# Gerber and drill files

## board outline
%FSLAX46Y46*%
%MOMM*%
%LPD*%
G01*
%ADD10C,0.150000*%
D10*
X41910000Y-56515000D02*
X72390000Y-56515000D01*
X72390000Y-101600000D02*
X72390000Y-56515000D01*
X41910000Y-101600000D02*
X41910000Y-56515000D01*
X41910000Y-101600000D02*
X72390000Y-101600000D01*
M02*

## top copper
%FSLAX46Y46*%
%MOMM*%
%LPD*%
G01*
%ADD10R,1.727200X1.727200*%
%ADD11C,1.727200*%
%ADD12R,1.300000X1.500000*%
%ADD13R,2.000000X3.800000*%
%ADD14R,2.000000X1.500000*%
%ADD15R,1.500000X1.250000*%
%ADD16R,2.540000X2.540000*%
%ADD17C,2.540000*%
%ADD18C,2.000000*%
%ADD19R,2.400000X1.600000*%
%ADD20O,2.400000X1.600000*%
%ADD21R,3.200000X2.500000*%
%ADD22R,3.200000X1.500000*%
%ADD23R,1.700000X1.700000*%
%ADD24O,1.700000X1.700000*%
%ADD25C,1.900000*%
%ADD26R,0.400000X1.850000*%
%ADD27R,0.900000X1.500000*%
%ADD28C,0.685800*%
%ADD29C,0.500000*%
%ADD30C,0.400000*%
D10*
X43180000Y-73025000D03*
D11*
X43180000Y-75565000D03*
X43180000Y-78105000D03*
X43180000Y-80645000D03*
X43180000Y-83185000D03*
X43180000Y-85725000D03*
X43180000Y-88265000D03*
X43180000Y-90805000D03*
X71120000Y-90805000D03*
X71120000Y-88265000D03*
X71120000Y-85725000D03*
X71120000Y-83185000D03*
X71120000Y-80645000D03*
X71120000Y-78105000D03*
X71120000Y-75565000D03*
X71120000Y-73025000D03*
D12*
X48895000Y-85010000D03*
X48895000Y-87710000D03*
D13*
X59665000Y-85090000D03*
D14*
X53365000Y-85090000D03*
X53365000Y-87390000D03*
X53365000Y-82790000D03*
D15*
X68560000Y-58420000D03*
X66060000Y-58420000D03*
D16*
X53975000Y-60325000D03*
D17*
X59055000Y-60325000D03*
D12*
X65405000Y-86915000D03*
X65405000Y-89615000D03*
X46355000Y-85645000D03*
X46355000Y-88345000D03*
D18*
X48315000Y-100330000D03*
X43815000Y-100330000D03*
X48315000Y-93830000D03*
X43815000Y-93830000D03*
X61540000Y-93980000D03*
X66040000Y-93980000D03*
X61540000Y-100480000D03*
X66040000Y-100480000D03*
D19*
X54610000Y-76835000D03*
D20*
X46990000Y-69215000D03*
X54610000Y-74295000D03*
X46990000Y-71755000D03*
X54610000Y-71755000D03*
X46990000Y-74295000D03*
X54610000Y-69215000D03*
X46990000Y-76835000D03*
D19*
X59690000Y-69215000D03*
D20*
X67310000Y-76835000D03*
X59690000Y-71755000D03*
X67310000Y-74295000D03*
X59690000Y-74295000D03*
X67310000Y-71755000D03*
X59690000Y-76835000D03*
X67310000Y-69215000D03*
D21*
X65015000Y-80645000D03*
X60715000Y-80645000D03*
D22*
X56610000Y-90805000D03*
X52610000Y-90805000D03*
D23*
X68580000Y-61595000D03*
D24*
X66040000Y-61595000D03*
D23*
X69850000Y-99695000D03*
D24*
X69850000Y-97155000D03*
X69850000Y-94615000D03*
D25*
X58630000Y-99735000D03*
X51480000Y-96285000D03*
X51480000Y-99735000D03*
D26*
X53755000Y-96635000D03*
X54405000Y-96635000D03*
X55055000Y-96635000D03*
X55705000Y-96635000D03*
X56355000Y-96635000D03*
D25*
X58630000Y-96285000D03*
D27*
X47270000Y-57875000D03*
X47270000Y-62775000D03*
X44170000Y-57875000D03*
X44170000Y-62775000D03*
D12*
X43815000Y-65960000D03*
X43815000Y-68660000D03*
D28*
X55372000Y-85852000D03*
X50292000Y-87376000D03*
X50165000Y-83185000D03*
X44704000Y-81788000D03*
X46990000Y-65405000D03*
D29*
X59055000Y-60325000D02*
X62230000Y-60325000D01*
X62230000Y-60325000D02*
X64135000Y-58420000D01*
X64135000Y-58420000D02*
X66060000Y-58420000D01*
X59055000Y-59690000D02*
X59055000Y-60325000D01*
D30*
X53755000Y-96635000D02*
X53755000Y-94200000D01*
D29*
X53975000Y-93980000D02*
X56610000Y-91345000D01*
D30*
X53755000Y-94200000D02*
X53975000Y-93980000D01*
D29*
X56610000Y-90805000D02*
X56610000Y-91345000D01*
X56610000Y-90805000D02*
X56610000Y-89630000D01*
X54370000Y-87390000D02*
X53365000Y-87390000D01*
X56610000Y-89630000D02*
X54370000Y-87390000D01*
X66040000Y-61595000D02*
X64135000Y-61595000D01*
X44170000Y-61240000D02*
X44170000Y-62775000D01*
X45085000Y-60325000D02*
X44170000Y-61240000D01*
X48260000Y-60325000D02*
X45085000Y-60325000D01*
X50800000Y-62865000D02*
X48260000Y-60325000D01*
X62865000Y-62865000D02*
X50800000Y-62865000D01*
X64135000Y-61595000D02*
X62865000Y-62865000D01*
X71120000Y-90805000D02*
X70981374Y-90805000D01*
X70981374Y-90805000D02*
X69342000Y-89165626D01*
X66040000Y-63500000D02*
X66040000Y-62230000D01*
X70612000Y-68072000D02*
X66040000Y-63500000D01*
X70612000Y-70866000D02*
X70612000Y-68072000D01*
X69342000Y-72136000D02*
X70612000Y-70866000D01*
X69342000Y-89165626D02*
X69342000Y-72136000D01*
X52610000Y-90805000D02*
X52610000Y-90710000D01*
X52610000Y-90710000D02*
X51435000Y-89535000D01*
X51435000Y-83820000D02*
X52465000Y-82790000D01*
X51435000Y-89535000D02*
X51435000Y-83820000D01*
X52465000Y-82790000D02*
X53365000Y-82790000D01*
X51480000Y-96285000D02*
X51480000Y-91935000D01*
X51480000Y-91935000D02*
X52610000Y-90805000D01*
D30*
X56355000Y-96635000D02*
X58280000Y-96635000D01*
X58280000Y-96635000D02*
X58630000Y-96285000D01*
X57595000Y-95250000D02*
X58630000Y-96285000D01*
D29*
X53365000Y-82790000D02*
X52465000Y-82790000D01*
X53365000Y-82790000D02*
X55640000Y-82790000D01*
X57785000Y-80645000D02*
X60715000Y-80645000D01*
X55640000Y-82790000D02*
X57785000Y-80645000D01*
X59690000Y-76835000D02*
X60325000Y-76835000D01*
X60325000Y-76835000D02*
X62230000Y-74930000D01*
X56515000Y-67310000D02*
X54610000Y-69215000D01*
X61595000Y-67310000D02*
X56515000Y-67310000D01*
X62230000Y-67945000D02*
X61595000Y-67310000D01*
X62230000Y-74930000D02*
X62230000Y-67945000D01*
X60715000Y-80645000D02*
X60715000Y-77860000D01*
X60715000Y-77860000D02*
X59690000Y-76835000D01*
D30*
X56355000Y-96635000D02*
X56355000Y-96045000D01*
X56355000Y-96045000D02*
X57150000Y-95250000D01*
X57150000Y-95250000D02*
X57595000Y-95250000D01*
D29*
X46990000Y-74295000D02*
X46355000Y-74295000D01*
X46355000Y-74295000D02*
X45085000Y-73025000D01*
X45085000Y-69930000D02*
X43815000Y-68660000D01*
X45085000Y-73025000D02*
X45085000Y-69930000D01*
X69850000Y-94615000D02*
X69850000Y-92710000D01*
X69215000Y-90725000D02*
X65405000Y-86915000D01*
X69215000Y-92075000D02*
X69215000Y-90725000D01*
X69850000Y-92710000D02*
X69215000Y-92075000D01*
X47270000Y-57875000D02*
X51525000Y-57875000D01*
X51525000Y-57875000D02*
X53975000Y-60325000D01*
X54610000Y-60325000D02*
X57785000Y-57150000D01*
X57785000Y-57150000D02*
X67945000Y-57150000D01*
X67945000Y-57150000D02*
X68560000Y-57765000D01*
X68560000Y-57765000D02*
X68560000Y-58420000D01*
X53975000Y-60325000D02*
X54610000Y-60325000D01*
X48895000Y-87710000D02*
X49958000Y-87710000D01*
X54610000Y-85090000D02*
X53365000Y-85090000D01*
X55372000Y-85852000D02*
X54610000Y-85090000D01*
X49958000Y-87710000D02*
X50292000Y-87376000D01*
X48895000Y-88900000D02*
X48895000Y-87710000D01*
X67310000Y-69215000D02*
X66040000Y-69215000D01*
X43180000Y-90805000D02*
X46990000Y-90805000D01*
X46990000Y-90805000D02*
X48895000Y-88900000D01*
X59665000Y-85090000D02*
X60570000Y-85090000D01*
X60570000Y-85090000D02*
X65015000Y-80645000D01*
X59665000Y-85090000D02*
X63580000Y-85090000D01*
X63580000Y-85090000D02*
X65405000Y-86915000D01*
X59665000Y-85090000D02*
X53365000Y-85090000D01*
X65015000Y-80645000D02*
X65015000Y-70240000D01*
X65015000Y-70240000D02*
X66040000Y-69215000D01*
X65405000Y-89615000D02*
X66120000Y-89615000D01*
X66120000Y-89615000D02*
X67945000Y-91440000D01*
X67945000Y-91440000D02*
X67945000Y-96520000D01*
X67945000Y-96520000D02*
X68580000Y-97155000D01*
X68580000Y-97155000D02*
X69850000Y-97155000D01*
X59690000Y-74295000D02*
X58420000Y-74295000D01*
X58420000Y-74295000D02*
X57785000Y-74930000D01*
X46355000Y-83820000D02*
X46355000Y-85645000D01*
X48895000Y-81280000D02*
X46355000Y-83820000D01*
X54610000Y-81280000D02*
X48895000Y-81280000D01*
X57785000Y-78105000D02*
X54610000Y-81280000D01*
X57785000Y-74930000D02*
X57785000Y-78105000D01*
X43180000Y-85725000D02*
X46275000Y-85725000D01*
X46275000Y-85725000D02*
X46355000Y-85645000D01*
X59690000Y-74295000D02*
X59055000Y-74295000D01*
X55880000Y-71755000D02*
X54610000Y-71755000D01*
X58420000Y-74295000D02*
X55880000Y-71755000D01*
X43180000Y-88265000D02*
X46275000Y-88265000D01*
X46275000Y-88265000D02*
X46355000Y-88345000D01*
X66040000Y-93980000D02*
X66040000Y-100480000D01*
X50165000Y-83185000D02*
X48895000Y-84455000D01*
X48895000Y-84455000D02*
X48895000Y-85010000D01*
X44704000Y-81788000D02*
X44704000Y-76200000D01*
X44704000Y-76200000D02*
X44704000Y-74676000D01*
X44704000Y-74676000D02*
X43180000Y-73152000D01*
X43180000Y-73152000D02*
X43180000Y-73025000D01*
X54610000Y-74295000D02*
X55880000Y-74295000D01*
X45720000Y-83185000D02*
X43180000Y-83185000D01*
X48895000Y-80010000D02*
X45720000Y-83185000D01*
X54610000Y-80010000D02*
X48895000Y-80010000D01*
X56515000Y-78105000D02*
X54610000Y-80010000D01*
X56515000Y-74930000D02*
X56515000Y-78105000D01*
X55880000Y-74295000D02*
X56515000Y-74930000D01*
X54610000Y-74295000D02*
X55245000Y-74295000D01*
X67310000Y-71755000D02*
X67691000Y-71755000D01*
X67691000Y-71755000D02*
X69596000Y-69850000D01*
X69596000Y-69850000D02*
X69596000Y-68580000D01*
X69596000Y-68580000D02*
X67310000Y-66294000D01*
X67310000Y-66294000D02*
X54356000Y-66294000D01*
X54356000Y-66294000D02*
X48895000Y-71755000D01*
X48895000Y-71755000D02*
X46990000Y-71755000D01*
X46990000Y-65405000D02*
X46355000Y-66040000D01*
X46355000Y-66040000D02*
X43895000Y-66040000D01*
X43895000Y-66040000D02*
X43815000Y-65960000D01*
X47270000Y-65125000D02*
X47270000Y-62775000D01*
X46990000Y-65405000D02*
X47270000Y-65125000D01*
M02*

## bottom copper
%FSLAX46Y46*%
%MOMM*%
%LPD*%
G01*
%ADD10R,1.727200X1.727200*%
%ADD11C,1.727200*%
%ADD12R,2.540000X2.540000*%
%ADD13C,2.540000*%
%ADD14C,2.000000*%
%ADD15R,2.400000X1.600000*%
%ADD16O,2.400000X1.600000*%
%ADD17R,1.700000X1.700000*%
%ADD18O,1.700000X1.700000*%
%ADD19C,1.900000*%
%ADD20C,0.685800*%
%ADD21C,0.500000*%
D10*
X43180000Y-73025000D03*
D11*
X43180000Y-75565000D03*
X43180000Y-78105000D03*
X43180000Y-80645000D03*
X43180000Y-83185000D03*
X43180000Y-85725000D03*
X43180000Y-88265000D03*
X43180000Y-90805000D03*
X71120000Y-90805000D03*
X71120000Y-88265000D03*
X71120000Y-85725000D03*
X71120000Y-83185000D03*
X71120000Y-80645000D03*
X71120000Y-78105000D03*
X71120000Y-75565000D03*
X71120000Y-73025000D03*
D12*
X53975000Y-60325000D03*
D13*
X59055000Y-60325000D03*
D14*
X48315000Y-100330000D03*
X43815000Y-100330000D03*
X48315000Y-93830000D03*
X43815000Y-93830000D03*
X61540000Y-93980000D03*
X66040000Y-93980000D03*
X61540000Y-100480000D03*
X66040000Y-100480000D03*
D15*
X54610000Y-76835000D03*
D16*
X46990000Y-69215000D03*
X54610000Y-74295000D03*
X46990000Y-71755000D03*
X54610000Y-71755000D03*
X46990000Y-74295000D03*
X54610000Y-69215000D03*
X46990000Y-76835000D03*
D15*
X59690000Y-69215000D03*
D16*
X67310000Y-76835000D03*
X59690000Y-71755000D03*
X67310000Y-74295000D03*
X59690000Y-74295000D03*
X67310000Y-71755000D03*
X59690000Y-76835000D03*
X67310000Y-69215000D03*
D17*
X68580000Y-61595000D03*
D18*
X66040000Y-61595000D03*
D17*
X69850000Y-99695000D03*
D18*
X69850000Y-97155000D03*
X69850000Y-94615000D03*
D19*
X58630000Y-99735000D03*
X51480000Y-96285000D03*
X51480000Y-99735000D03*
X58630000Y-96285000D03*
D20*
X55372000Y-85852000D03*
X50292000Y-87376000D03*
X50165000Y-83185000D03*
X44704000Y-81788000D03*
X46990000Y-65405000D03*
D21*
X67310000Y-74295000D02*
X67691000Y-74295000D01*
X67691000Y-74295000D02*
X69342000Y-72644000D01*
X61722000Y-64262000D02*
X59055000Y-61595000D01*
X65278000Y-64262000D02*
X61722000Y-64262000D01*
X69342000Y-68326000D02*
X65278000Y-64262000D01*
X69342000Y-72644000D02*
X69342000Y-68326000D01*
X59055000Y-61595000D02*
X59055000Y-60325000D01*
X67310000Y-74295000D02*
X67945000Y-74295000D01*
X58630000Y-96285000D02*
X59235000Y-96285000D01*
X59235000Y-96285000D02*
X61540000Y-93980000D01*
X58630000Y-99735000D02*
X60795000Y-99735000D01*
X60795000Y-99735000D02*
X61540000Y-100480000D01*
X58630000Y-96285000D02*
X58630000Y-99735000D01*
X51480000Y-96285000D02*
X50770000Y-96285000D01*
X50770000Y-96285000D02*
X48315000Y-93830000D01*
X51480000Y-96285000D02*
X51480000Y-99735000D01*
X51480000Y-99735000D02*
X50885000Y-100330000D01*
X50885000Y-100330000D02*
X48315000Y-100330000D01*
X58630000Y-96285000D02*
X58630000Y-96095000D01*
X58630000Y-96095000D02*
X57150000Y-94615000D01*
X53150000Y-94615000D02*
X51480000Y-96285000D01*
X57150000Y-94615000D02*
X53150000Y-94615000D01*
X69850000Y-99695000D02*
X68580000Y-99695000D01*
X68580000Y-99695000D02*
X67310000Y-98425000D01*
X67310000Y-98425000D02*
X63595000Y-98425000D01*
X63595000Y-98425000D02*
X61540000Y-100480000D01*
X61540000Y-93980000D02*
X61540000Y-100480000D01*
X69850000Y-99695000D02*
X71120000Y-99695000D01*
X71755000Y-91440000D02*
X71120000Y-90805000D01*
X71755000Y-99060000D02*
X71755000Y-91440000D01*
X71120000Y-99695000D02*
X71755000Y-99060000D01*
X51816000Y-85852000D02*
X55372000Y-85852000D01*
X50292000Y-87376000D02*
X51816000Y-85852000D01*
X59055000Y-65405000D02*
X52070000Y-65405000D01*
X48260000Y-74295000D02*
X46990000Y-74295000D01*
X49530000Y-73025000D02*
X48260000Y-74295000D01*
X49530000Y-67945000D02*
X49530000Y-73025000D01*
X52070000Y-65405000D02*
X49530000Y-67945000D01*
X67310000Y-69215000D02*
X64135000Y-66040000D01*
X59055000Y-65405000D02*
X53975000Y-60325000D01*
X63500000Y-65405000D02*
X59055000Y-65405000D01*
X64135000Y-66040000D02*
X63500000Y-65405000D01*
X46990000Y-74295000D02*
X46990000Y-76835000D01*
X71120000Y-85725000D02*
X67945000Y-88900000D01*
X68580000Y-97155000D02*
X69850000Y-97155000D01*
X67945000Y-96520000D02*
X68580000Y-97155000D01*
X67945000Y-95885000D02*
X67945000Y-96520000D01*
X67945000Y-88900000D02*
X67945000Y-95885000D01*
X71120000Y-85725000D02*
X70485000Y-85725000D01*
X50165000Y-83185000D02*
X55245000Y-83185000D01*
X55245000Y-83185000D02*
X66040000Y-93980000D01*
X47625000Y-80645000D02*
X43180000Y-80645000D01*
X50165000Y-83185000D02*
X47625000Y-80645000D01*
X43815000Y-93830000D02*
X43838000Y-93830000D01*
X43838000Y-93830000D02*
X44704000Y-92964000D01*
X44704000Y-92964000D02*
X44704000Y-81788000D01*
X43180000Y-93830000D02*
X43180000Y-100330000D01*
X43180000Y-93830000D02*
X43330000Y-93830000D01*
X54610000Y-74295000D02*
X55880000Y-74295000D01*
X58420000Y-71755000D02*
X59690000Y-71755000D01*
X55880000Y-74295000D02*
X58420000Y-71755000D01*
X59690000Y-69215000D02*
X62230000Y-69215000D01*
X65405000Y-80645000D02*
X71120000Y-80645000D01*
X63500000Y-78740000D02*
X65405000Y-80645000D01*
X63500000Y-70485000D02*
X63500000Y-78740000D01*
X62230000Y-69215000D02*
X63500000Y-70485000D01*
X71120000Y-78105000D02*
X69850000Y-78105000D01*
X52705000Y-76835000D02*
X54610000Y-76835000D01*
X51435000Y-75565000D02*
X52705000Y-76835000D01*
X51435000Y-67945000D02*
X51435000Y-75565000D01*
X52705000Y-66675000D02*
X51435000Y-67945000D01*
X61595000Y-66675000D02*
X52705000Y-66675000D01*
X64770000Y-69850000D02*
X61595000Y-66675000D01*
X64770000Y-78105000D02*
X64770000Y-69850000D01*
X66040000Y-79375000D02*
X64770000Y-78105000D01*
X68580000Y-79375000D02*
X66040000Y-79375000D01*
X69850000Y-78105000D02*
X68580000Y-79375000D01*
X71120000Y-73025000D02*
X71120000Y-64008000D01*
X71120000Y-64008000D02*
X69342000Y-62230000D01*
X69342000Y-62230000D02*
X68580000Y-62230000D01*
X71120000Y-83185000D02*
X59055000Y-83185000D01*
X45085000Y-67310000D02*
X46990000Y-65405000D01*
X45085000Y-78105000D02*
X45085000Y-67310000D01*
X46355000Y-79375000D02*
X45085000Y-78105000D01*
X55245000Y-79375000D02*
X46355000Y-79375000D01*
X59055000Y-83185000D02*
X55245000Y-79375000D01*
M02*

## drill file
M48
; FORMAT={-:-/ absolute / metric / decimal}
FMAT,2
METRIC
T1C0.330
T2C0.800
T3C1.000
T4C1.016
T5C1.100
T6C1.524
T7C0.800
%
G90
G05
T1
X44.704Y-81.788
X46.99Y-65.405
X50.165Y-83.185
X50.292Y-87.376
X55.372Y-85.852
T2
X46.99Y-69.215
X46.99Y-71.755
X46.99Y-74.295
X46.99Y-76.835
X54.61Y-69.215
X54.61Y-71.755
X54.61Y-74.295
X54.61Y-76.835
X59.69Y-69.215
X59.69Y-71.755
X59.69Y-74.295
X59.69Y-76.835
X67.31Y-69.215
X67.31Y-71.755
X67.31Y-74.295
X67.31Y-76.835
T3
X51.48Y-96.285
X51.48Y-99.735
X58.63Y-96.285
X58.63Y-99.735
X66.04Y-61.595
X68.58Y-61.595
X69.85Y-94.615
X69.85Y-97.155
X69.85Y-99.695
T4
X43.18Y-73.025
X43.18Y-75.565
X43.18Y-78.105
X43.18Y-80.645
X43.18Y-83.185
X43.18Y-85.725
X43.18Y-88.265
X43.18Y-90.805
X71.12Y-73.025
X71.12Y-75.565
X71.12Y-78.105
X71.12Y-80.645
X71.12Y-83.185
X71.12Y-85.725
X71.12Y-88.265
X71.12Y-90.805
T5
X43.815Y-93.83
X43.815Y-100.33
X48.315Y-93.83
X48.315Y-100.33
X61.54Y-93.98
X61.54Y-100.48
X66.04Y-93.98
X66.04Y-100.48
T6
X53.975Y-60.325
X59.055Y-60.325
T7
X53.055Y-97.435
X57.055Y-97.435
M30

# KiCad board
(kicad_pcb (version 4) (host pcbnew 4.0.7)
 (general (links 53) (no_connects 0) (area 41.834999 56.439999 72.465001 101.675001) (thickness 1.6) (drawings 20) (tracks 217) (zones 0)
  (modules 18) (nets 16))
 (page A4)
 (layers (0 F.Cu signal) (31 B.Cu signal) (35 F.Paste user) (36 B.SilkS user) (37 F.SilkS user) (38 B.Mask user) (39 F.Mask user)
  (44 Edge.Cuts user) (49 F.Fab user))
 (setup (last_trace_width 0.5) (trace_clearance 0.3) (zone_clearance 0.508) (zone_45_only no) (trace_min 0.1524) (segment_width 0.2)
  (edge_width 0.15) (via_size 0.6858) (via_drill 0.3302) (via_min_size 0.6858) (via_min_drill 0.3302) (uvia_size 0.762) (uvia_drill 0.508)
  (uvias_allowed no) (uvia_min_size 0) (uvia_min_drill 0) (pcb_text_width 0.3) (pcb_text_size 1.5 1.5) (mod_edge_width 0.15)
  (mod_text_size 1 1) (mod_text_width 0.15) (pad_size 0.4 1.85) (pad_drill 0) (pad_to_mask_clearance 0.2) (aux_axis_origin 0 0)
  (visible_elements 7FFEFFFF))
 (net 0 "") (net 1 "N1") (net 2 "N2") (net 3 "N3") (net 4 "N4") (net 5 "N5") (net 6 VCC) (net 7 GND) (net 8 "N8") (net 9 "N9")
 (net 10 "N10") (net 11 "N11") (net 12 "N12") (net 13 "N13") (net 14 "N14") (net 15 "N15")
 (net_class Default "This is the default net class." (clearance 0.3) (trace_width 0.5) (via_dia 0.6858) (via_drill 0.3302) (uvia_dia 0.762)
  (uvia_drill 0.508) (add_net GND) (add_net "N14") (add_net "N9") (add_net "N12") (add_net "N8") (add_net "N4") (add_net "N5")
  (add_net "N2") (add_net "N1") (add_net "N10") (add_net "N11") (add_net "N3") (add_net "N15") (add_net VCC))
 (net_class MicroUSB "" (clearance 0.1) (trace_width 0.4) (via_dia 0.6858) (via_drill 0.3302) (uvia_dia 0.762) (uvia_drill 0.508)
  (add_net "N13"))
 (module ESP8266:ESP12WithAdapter (layer F.Cu) (at 41.91 92.075)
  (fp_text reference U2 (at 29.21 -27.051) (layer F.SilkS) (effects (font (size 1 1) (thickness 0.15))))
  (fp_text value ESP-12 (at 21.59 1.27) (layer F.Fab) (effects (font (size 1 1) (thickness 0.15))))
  (pad 1 thru_hole rect (at 1.27 -19.05) (size 1.7272 1.7272) (drill 1.016) (layers *.Cu *.Mask F.SilkS) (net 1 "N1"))
  (pad 2 thru_hole circle (at 1.27 -16.51) (size 1.7272 1.7272) (drill 1.016) (layers *.Cu *.Mask F.SilkS))
  (pad 3 thru_hole circle (at 1.27 -13.97) (size 1.7272 1.7272) (drill 1.016) (layers *.Cu *.Mask F.SilkS))
  (pad 4 thru_hole circle (at 1.27 -11.43) (size 1.7272 1.7272) (drill 1.016) (layers *.Cu *.Mask F.SilkS) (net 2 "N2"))
  (pad 5 thru_hole circle (at 1.27 -8.89) (size 1.7272 1.7272) (drill 1.016) (layers *.Cu *.Mask F.SilkS) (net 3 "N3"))
  (pad 6 thru_hole circle (at 1.27 -6.35) (size 1.7272 1.7272) (drill 1.016) (layers *.Cu *.Mask F.SilkS) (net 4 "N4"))
  (pad 7 thru_hole circle (at 1.27 -3.81) (size 1.7272 1.7272) (drill 1.016) (layers *.Cu *.Mask F.SilkS) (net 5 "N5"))
  (pad 8 thru_hole circle (at 1.27 -1.27) (size 1.7272 1.7272) (drill 1.016) (layers *.Cu *.Mask F.SilkS) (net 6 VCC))
  (pad 9 thru_hole circle (at 29.21 -1.27) (size 1.7272 1.7272) (drill 1.016) (layers *.Cu *.Mask F.SilkS) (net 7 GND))
  (pad 10 thru_hole circle (at 29.21 -3.81) (size 1.7272 1.7272) (drill 1.016) (layers *.Cu *.Mask F.SilkS))
  (pad 11 thru_hole circle (at 29.21 -6.35) (size 1.7272 1.7272) (drill 1.016) (layers *.Cu *.Mask F.SilkS) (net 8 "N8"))
  (pad 12 thru_hole circle (at 29.21 -8.89) (size 1.7272 1.7272) (drill 1.016) (layers *.Cu *.Mask F.SilkS) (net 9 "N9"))
  (pad 13 thru_hole circle (at 29.21 -11.43) (size 1.7272 1.7272) (drill 1.016) (layers *.Cu *.Mask F.SilkS) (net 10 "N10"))
  (pad 14 thru_hole circle (at 29.21 -13.97) (size 1.7272 1.7272) (drill 1.016) (layers *.Cu *.Mask F.SilkS) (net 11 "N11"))
  (pad 15 thru_hole circle (at 29.21 -16.51) (size 1.7272 1.7272) (drill 1.016) (layers *.Cu *.Mask F.SilkS))
  (pad 16 thru_hole circle (at 29.21 -19.05) (size 1.7272 1.7272) (drill 1.016) (layers *.Cu *.Mask F.SilkS) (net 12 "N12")))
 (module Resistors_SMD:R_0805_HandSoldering (layer F.Cu) (at 48.895 86.36 270)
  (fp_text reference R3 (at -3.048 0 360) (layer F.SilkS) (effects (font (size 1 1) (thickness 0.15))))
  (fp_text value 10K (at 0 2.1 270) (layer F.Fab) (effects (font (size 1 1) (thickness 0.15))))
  (pad 1 smd rect (at -1.35 0 270) (size 1.5 1.3) (layers F.Cu F.Paste F.Mask) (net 2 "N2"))
  (pad 2 smd rect (at 1.35 0 270) (size 1.5 1.3) (layers F.Cu F.Paste F.Mask) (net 6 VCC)))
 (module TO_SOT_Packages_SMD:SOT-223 (layer F.Cu) (at 56.515 85.09)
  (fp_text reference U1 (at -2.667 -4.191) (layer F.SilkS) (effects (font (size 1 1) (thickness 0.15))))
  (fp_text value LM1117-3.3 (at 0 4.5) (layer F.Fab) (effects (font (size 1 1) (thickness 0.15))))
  (pad 2 smd rect (at 3.15 0) (size 2 3.8) (layers F.Cu F.Paste F.Mask) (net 6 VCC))
  (pad 2 smd rect (at -3.15 0) (size 2 1.5) (layers F.Cu F.Paste F.Mask) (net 6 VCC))
  (pad 3 smd rect (at -3.15 2.3) (size 2 1.5) (layers F.Cu F.Paste F.Mask) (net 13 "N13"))
  (pad 1 smd rect (at -3.15 -2.3) (size 2 1.5) (layers F.Cu F.Paste F.Mask) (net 7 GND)))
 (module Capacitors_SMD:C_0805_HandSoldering (layer F.Cu) (at 67.31 58.42 180)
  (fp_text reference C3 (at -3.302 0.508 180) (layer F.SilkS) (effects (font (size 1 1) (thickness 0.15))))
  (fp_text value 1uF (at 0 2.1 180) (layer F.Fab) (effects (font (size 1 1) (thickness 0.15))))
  (pad 1 smd rect (at -1.25 0 180) (size 1.5 1.25) (layers F.Cu F.Paste F.Mask) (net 6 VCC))
  (pad 2 smd rect (at 1.25 0 180) (size 1.5 1.25) (layers F.Cu F.Paste F.Mask) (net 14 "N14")))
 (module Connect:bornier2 (layer F.Cu) (at 56.515 60.325)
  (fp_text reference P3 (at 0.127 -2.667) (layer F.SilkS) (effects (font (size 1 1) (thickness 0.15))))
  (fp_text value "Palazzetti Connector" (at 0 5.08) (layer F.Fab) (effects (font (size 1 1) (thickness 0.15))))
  (pad 1 thru_hole rect (at -2.54 0) (size 2.54 2.54) (drill 1.524) (layers *.Cu *.Mask) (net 6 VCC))
  (pad 2 thru_hole circle (at 2.54 0) (size 2.54 2.54) (drill 1.524) (layers *.Cu *.Mask) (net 14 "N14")))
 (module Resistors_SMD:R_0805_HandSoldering (layer F.Cu) (at 65.405 88.265 270)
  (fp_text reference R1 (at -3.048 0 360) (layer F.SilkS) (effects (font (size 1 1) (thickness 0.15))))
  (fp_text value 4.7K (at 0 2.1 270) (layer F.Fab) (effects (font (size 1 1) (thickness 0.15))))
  (pad 1 smd rect (at -1.35 0 270) (size 1.5 1.3) (layers F.Cu F.Paste F.Mask) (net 6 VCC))
  (pad 2 smd rect (at 1.35 0 270) (size 1.5 1.3) (layers F.Cu F.Paste F.Mask) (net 8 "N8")))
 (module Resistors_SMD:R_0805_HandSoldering (layer F.Cu) (at 46.355 86.995 270)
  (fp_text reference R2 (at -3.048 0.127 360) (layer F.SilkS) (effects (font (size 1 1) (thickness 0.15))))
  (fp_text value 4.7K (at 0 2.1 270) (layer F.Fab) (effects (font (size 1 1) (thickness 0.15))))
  (pad 1 smd rect (at -1.35 0 270) (size 1.5 1.3) (layers F.Cu F.Paste F.Mask) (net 4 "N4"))
  (pad 2 smd rect (at 1.35 0 270) (size 1.5 1.3) (layers F.Cu F.Paste F.Mask) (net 5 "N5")))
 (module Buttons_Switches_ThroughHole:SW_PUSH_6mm (layer F.Cu) (at 43.815 100.33 90)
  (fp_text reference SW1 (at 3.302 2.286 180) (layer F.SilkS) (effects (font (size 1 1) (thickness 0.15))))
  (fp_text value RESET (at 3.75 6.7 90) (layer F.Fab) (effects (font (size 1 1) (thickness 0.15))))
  (pad 2 thru_hole circle (at 0 4.5 180) (size 2 2) (drill 1.1) (layers *.Cu *.Mask) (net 7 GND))
  (pad 1 thru_hole circle (at 0 0 180) (size 2 2) (drill 1.1) (layers *.Cu *.Mask) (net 1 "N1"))
  (pad 2 thru_hole circle (at 6.5 4.5 180) (size 2 2) (drill 1.1) (layers *.Cu *.Mask) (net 7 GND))
  (pad 1 thru_hole circle (at 6.5 0 180) (size 2 2) (drill 1.1) (layers *.Cu *.Mask) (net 1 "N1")))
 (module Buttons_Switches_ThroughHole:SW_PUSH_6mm (layer F.Cu) (at 66.04 93.98 270)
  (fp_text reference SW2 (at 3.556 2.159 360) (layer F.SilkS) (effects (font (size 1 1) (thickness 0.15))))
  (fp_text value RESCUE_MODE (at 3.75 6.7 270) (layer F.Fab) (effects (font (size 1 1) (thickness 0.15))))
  (pad 2 thru_hole circle (at 0 4.5) (size 2 2) (drill 1.1) (layers *.Cu *.Mask) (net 7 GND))
  (pad 1 thru_hole circle (at 0 0) (size 2 2) (drill 1.1) (layers *.Cu *.Mask) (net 2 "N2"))
  (pad 2 thru_hole circle (at 6.5 4.5) (size 2 2) (drill 1.1) (layers *.Cu *.Mask) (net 7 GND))
  (pad 1 thru_hole circle (at 6.5 0) (size 2 2) (drill 1.1) (layers *.Cu *.Mask) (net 2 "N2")))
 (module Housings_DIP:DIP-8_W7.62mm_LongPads (layer F.Cu) (at 54.61 76.835 180)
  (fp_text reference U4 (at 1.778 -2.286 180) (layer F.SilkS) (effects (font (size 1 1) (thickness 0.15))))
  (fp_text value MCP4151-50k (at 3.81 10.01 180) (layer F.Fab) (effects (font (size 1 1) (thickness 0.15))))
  (pad 1 thru_hole rect (at 0 0 180) (size 2.4 1.6) (drill 0.8) (layers *.Cu *.Mask) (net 11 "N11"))
  (pad 5 thru_hole oval (at 7.62 7.62 180) (size 2.4 1.6) (drill 0.8) (layers *.Cu *.Mask))
  (pad 2 thru_hole oval (at 0 2.54 180) (size 2.4 1.6) (drill 0.8) (layers *.Cu *.Mask) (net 3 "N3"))
  (pad 6 thru_hole oval (at 7.62 5.08 180) (size 2.4 1.6) (drill 0.8) (layers *.Cu *.Mask) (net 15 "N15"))
  (pad 3 thru_hole oval (at 0 5.08 180) (size 2.4 1.6) (drill 0.8) (layers *.Cu *.Mask) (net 4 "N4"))
  (pad 7 thru_hole oval (at 7.62 2.54 180) (size 2.4 1.6) (drill 0.8) (layers *.Cu *.Mask) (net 6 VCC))
  (pad 4 thru_hole oval (at 0 7.62 180) (size 2.4 1.6) (drill 0.8) (layers *.Cu *.Mask) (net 7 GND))
  (pad 8 thru_hole oval (at 7.62 0 180) (size 2.4 1.6) (drill 0.8) (layers *.Cu *.Mask) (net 6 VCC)))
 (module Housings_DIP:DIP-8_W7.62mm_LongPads (layer F.Cu) (at 59.69 69.215)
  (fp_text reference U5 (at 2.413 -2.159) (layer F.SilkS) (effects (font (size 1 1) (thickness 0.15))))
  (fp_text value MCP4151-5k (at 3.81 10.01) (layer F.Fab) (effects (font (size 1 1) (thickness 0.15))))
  (pad 1 thru_hole rect (at 0 0) (size 2.4 1.6) (drill 0.8) (layers *.Cu *.Mask) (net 10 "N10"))
  (pad 5 thru_hole oval (at 7.62 7.62) (size 2.4 1.6) (drill 0.8) (layers *.Cu *.Mask))
  (pad 2 thru_hole oval (at 0 2.54) (size 2.4 1.6) (drill 0.8) (layers *.Cu *.Mask) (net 3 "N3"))
  (pad 6 thru_hole oval (at 7.62 5.08) (size 2.4 1.6) (drill 0.8) (layers *.Cu *.Mask) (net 14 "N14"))
  (pad 3 thru_hole oval (at 0 5.08) (size 2.4 1.6) (drill 0.8) (layers *.Cu *.Mask) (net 4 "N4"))
  (pad 7 thru_hole oval (at 7.62 2.54) (size 2.4 1.6) (drill 0.8) (layers *.Cu *.Mask) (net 15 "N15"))
  (pad 4 thru_hole oval (at 0 7.62) (size 2.4 1.6) (drill 0.8) (layers *.Cu *.Mask) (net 7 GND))
  (pad 8 thru_hole oval (at 7.62 0) (size 2.4 1.6) (drill 0.8) (layers *.Cu *.Mask) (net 6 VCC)))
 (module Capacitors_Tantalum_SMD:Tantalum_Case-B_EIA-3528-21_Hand (layer F.Cu) (at 62.865 80.645 180)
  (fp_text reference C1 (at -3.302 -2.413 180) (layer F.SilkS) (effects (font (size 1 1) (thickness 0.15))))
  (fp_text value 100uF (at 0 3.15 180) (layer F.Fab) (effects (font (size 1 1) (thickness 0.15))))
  (pad 1 smd rect (at -2.15 0 180) (size 3.2 2.5) (layers F.Cu F.Paste F.Mask) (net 6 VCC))
  (pad 2 smd rect (at 2.15 0 180) (size 3.2 2.5) (layers F.Cu F.Paste F.Mask) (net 7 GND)))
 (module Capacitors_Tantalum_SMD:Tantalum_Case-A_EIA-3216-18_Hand (layer F.Cu) (at 54.61 90.805 180)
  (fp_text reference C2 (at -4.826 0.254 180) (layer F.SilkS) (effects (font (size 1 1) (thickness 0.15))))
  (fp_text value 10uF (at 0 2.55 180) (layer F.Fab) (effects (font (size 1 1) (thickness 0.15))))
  (pad 1 smd rect (at -2 0 180) (size 3.2 1.5) (layers F.Cu F.Paste F.Mask) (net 13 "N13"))
  (pad 2 smd rect (at 2 0 180) (size 3.2 1.5) (layers F.Cu F.Paste F.Mask) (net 7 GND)))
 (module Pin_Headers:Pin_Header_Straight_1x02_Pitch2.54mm (layer F.Cu) (at 68.58 61.595 270)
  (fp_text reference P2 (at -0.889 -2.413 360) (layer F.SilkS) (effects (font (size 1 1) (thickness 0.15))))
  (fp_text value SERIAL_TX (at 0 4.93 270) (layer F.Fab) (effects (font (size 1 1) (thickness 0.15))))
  (pad 1 thru_hole rect (at 0 0 270) (size 1.7 1.7) (drill 1) (layers *.Cu *.Mask) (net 12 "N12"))
  (pad 2 thru_hole oval (at 0 2.54 270) (size 1.7 1.7) (drill 1) (layers *.Cu *.Mask) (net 7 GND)))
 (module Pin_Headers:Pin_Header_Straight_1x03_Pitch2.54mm (layer F.Cu) (at 69.85 99.695 180)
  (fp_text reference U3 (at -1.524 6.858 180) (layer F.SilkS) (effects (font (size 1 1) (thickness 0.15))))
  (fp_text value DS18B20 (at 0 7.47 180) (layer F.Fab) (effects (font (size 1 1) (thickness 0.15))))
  (pad 1 thru_hole rect (at 0 0 180) (size 1.7 1.7) (drill 1) (layers *.Cu *.Mask) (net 7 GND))
  (pad 2 thru_hole oval (at 0 2.54 180) (size 1.7 1.7) (drill 1) (layers *.Cu *.Mask) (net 8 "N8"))
  (pad 3 thru_hole oval (at 0 5.08 180) (size 1.7 1.7) (drill 1) (layers *.Cu *.Mask) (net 6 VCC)))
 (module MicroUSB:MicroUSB (layer F.Cu) (at 59.055 95.885 180)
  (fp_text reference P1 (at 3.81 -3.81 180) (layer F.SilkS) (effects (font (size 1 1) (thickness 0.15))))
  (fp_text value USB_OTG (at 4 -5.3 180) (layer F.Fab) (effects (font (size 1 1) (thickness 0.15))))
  (pad 6 thru_hole circle (at 0.425 -3.85 180) (size 1.9 1.9) (drill 1) (layers *.Cu *.Mask F.SilkS) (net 7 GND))
  (pad 6 thru_hole circle (at 7.575 -0.4 180) (size 1.9 1.9) (drill 1) (layers *.Cu *.Mask F.SilkS) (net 7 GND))
  (pad 6 thru_hole circle (at 7.575 -3.85 180) (size 1.9 1.9) (drill 1) (layers *.Cu *.Mask F.SilkS) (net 7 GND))
  (pad 1 smd rect (at 5.3 -0.75 180) (size 0.4 1.85) (layers F.Cu F.Paste F.Mask) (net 13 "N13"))
  (pad 2 smd rect (at 4.65 -0.75 180) (size 0.4 1.85) (layers F.Cu F.Paste F.Mask))
  (pad 3 smd rect (at 4 -0.75 180) (size 0.4 1.85) (layers F.Cu F.Paste F.Mask))
  (pad 4 smd rect (at 3.35 -0.75 180) (size 0.4 1.85) (layers F.Cu F.Paste F.Mask))
  (pad "" np_thru_hole circle (at 6 -1.55 180) (size 0.8 0.8) (drill 0.8) (layers *.Cu *.Mask F.SilkS))
  (pad "" np_thru_hole circle (at 2 -1.55 180) (size 0.8 0.8) (drill 0.8) (layers *.Cu *.Mask F.SilkS))
  (pad 5 smd rect (at 2.7 -0.75 180) (size 0.4 1.85) (layers F.Cu F.Paste F.Mask) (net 7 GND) (clearance 0.1))
  (pad 6 thru_hole circle (at 0.425 -0.4 180) (size 1.9 1.9) (drill 1) (layers *.Cu *.Mask F.SilkS) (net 7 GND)))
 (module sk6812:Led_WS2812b (layer F.Cu) (at 45.72 60.325 270)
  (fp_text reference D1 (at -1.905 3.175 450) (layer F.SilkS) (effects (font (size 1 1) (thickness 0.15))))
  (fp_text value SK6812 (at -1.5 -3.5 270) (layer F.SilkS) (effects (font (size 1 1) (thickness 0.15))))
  (pad 1 smd rect (at -2.45 -1.55 270) (size 1.5 0.9) (layers F.Cu F.Paste F.Mask) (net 6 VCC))
  (pad 4 smd rect (at 2.45 -1.55 270) (size 1.5 0.9) (layers F.Cu F.Paste F.Mask) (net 9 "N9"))
  (pad 2 smd rect (at -2.45 1.55 270) (size 1.5 0.9) (layers F.Cu F.Paste F.Mask))
  (pad 3 smd rect (at 2.45 1.55 270) (size 1.5 0.9) (layers F.Cu F.Paste F.Mask) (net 7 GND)))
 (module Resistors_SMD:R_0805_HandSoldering (layer F.Cu) (at 43.815 67.31 270)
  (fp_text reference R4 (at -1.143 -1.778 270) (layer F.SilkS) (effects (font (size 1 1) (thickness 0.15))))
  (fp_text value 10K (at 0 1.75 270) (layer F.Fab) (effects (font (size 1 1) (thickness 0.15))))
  (pad 1 smd rect (at -1.35 0 270) (size 1.5 1.3) (layers F.Cu F.Paste F.Mask) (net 9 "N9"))
  (pad 2 smd rect (at 1.35 0 270) (size 1.5 1.3) (layers F.Cu F.Paste F.Mask) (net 6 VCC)))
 (gr_line (start 41.91 56.515) (end 72.39 56.515) (angle 90) (layer Edge.Cuts) (width 0.15))
 (gr_line (start 72.39 101.6) (end 72.39 56.515) (angle 90) (layer Edge.Cuts) (width 0.15))
 (gr_line (start 41.91 101.6) (end 41.91 56.515) (angle 90) (layer Edge.Cuts) (width 0.15))
 (gr_line (start 41.91 101.6) (end 72.39 101.6) (angle 90) (layer Edge.Cuts) (width 0.15))
 (segment (start 59.055 60.325) (end 62.23 60.325) (width 0.5) (layer F.Cu) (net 14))
 (segment (start 62.23 60.325) (end 64.135 58.42) (width 0.5) (layer F.Cu) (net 14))
 (segment (start 64.135 58.42) (end 66.06 58.42) (width 0.5) (layer F.Cu) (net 14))
 (segment (start 67.31 74.295) (end 67.691 74.295) (width 0.5) (layer B.Cu) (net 14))
 (segment (start 67.691 74.295) (end 69.342 72.644) (width 0.5) (layer B.Cu) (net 14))
 (segment (start 61.722 64.262) (end 59.055 61.595) (width 0.5) (layer B.Cu) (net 14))
 (segment (start 65.278 64.262) (end 61.722 64.262) (width 0.5) (layer B.Cu) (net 14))
 (segment (start 69.342 68.326) (end 65.278 64.262) (width 0.5) (layer B.Cu) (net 14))
 (segment (start 69.342 72.644) (end 69.342 68.326) (width 0.5) (layer B.Cu) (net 14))
 (segment (start 59.055 61.595) (end 59.055 60.325) (width 0.5) (layer B.Cu) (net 14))
 (segment (start 67.31 74.295) (end 67.945 74.295) (width 0.5) (layer B.Cu) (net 14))
 (segment (start 59.055 59.69) (end 59.055 60.325) (width 0.5) (layer F.Cu) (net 14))
 (segment (start 53.755 96.635) (end 53.755 94.2) (width 0.4) (layer F.Cu) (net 13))
 (segment (start 53.975 93.98) (end 56.61 91.345) (width 0.5) (layer F.Cu) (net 13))
 (segment (start 53.755 94.2) (end 53.975 93.98) (width 0.4) (layer F.Cu) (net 13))
 (segment (start 56.61 90.805) (end 56.61 91.345) (width 0.5) (layer F.Cu) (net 13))
 (segment (start 56.61 90.805) (end 56.61 89.63) (width 0.5) (layer F.Cu) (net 13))
 (segment (start 54.37 87.39) (end 53.365 87.39) (width 0.5) (layer F.Cu) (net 13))
 (segment (start 56.61 89.63) (end 54.37 87.39) (width 0.5) (layer F.Cu) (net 13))
 (segment (start 66.04 61.595) (end 64.135 61.595) (width 0.5) (layer F.Cu) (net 7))
 (segment (start 44.17 61.24) (end 44.17 62.775) (width 0.5) (layer F.Cu) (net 7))
 (segment (start 45.085 60.325) (end 44.17 61.24) (width 0.5) (layer F.Cu) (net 7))
 (segment (start 48.26 60.325) (end 45.085 60.325) (width 0.5) (layer F.Cu) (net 7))
 (segment (start 50.8 62.865) (end 48.26 60.325) (width 0.5) (layer F.Cu) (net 7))
 (segment (start 62.865 62.865) (end 50.8 62.865) (width 0.5) (layer F.Cu) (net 7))
 (segment (start 64.135 61.595) (end 62.865 62.865) (width 0.5) (layer F.Cu) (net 7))
 (segment (start 71.12 90.805) (end 70.981374 90.805) (width 0.5) (layer F.Cu) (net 7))
 (segment (start 70.981374 90.805) (end 69.342 89.165626) (width 0.5) (layer F.Cu) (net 7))
 (segment (start 66.04 63.5) (end 66.04 62.23) (width 0.5) (layer F.Cu) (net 7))
 (segment (start 70.612 68.072) (end 66.04 63.5) (width 0.5) (layer F.Cu) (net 7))
 (segment (start 70.612 70.866) (end 70.612 68.072) (width 0.5) (layer F.Cu) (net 7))
 (segment (start 69.342 72.136) (end 70.612 70.866) (width 0.5) (layer F.Cu) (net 7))
 (segment (start 69.342 89.165626) (end 69.342 72.136) (width 0.5) (layer F.Cu) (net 7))
 (segment (start 52.61 90.805) (end 52.61 90.71) (width 0.5) (layer F.Cu) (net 7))
 (segment (start 52.61 90.71) (end 51.435 89.535) (width 0.5) (layer F.Cu) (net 7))
 (segment (start 51.435 83.82) (end 52.465 82.79) (width 0.5) (layer F.Cu) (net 7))
 (segment (start 51.435 89.535) (end 51.435 83.82) (width 0.5) (layer F.Cu) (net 7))
 (segment (start 52.465 82.79) (end 53.365 82.79) (width 0.5) (layer F.Cu) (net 7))
 (segment (start 58.63 96.285) (end 59.235 96.285) (width 0.5) (layer B.Cu) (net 7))
 (segment (start 59.235 96.285) (end 61.54 93.98) (width 0.5) (layer B.Cu) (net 7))
 (segment (start 58.63 99.735) (end 60.795 99.735) (width 0.5) (layer B.Cu) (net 7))
 (segment (start 60.795 99.735) (end 61.54 100.48) (width 0.5) (layer B.Cu) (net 7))
 (segment (start 58.63 96.285) (end 58.63 99.735) (width 0.5) (layer B.Cu) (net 7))
 (segment (start 51.48 96.285) (end 50.77 96.285) (width 0.5) (layer B.Cu) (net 7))
 (segment (start 50.77 96.285) (end 48.315 93.83) (width 0.5) (layer B.Cu) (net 7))
 (segment (start 51.48 96.285) (end 51.48 99.735) (width 0.5) (layer B.Cu) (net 7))
 (segment (start 51.48 99.735) (end 50.885 100.33) (width 0.5) (layer B.Cu) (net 7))
 (segment (start 50.885 100.33) (end 48.315 100.33) (width 0.5) (layer B.Cu) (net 7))
 (segment (start 51.48 96.285) (end 51.48 91.935) (width 0.5) (layer F.Cu) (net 7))
 (segment (start 51.48 91.935) (end 52.61 90.805) (width 0.5) (layer F.Cu) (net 7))
 (segment (start 58.63 96.285) (end 58.63 96.095) (width 0.5) (layer B.Cu) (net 7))
 (segment (start 58.63 96.095) (end 57.15 94.615) (width 0.5) (layer B.Cu) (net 7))
 (segment (start 53.15 94.615) (end 51.48 96.285) (width 0.5) (layer B.Cu) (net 7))
 (segment (start 57.15 94.615) (end 53.15 94.615) (width 0.5) (layer B.Cu) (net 7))
 (segment (start 56.355 96.635) (end 58.28 96.635) (width 0.4) (layer F.Cu) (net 7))
 (segment (start 58.28 96.635) (end 58.63 96.285) (width 0.4) (layer F.Cu) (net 7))
 (segment (start 57.595 95.25) (end 58.63 96.285) (width 0.4) (layer F.Cu) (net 7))
 (segment (start 53.365 82.79) (end 52.465 82.79) (width 0.5) (layer F.Cu) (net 7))
 (segment (start 69.85 99.695) (end 68.58 99.695) (width 0.5) (layer B.Cu) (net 7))
 (segment (start 68.58 99.695) (end 67.31 98.425) (width 0.5) (layer B.Cu) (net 7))
 (segment (start 67.31 98.425) (end 63.595 98.425) (width 0.5) (layer B.Cu) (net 7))
 (segment (start 63.595 98.425) (end 61.54 100.48) (width 0.5) (layer B.Cu) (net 7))
 (segment (start 61.54 93.98) (end 61.54 100.48) (width 0.5) (layer B.Cu) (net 7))
 (segment (start 69.85 99.695) (end 71.12 99.695) (width 0.5) (layer B.Cu) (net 7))
 (segment (start 71.755 91.44) (end 71.12 90.805) (width 0.5) (layer B.Cu) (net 7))
 (segment (start 71.755 99.06) (end 71.755 91.44) (width 0.5) (layer B.Cu) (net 7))
 (segment (start 71.12 99.695) (end 71.755 99.06) (width 0.5) (layer B.Cu) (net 7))
 (segment (start 53.365 82.79) (end 55.64 82.79) (width 0.5) (layer F.Cu) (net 7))
 (segment (start 57.785 80.645) (end 60.715 80.645) (width 0.5) (layer F.Cu) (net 7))
 (segment (start 55.64 82.79) (end 57.785 80.645) (width 0.5) (layer F.Cu) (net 7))
 (segment (start 59.69 76.835) (end 60.325 76.835) (width 0.5) (layer F.Cu) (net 7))
 (segment (start 60.325 76.835) (end 62.23 74.93) (width 0.5) (layer F.Cu) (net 7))
 (segment (start 56.515 67.31) (end 54.61 69.215) (width 0.5) (layer F.Cu) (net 7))
 (segment (start 61.595 67.31) (end 56.515 67.31) (width 0.5) (layer F.Cu) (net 7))
 (segment (start 62.23 67.945) (end 61.595 67.31) (width 0.5) (layer F.Cu) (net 7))
 (segment (start 62.23 74.93) (end 62.23 67.945) (width 0.5) (layer F.Cu) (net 7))
 (segment (start 60.715 80.645) (end 60.715 77.86) (width 0.5) (layer F.Cu) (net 7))
 (segment (start 60.715 77.86) (end 59.69 76.835) (width 0.5) (layer F.Cu) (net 7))
 (segment (start 56.355 96.635) (end 56.355 96.045) (width 0.4) (layer F.Cu) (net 7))
 (segment (start 56.355 96.045) (end 57.15 95.25) (width 0.4) (layer F.Cu) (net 7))
 (segment (start 57.15 95.25) (end 57.595 95.25) (width 0.4) (layer F.Cu) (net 7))
 (segment (start 46.99 74.295) (end 46.355 74.295) (width 0.5) (layer F.Cu) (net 6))
 (segment (start 46.355 74.295) (end 45.085 73.025) (width 0.5) (layer F.Cu) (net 6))
 (segment (start 45.085 69.93) (end 43.815 68.66) (width 0.5) (layer F.Cu) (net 6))
 (segment (start 45.085 73.025) (end 45.085 69.93) (width 0.5) (layer F.Cu) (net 6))
 (segment (start 69.85 94.615) (end 69.85 92.71) (width 0.5) (layer F.Cu) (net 6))
 (segment (start 69.215 90.725) (end 65.405 86.915) (width 0.5) (layer F.Cu) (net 6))
 (segment (start 69.215 92.075) (end 69.215 90.725) (width 0.5) (layer F.Cu) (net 6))
 (segment (start 69.85 92.71) (end 69.215 92.075) (width 0.5) (layer F.Cu) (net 6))
 (segment (start 47.27 57.875) (end 51.525 57.875) (width 0.5) (layer F.Cu) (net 6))
 (segment (start 51.525 57.875) (end 53.975 60.325) (width 0.5) (layer F.Cu) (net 6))
 (segment (start 54.61 60.325) (end 57.785 57.15) (width 0.5) (layer F.Cu) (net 6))
 (segment (start 57.785 57.15) (end 67.945 57.15) (width 0.5) (layer F.Cu) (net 6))
 (segment (start 67.945 57.15) (end 68.56 57.765) (width 0.5) (layer F.Cu) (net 6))
 (segment (start 68.56 57.765) (end 68.56 58.42) (width 0.5) (layer F.Cu) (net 6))
 (segment (start 53.975 60.325) (end 54.61 60.325) (width 0.5) (layer F.Cu) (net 6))
 (segment (start 48.895 87.71) (end 49.958 87.71) (width 0.5) (layer F.Cu) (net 6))
 (segment (start 54.61 85.09) (end 53.365 85.09) (width 0.5) (layer F.Cu) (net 6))
 (segment (start 55.372 85.852) (end 54.61 85.09) (width 0.5) (layer F.Cu) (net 6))
 (via (at 55.372 85.852) (size 0.6858) (drill 0.3302) (layers F.Cu B.Cu) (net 6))
 (segment (start 51.816 85.852) (end 55.372 85.852) (width 0.5) (layer B.Cu) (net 6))
 (segment (start 50.292 87.376) (end 51.816 85.852) (width 0.5) (layer B.Cu) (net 6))
 (via (at 50.292 87.376) (size 0.6858) (drill 0.3302) (layers F.Cu B.Cu) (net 6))
 (segment (start 49.958 87.71) (end 50.292 87.376) (width 0.5) (layer F.Cu) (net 6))
 (segment (start 48.895 88.9) (end 48.895 87.71) (width 0.5) (layer F.Cu) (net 6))
 (segment (start 59.055 65.405) (end 52.07 65.405) (width 0.5) (layer B.Cu) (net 6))
 (segment (start 48.26 74.295) (end 46.99 74.295) (width 0.5) (layer B.Cu) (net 6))
 (segment (start 49.53 73.025) (end 48.26 74.295) (width 0.5) (layer B.Cu) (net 6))
 (segment (start 49.53 67.945) (end 49.53 73.025) (width 0.5) (layer B.Cu) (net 6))
 (segment (start 52.07 65.405) (end 49.53 67.945) (width 0.5) (layer B.Cu) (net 6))
 (segment (start 67.31 69.215) (end 66.04 69.215) (width 0.5) (layer F.Cu) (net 6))
 (segment (start 43.18 90.805) (end 46.99 90.805) (width 0.5) (layer F.Cu) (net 6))
 (segment (start 46.99 90.805) (end 48.895 88.9) (width 0.5) (layer F.Cu) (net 6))
 (segment (start 67.31 69.215) (end 64.135 66.04) (width 0.5) (layer B.Cu) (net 6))
 (segment (start 59.055 65.405) (end 53.975 60.325) (width 0.5) (layer B.Cu) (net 6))
 (segment (start 63.5 65.405) (end 59.055 65.405) (width 0.5) (layer B.Cu) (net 6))
 (segment (start 64.135 66.04) (end 63.5 65.405) (width 0.5) (layer B.Cu) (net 6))
 (segment (start 59.665 85.09) (end 60.57 85.09) (width 0.5) (layer F.Cu) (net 6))
 (segment (start 60.57 85.09) (end 65.015 80.645) (width 0.5) (layer F.Cu) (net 6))
 (segment (start 59.665 85.09) (end 63.58 85.09) (width 0.5) (layer F.Cu) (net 6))
 (segment (start 63.58 85.09) (end 65.405 86.915) (width 0.5) (layer F.Cu) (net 6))
 (segment (start 59.665 85.09) (end 53.365 85.09) (width 0.5) (layer F.Cu) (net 6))
 (segment (start 46.99 74.295) (end 46.99 76.835) (width 0.5) (layer B.Cu) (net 6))
 (segment (start 65.015 80.645) (end 65.015 70.24) (width 0.5) (layer F.Cu) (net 6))
 (segment (start 65.015 70.24) (end 66.04 69.215) (width 0.5) (layer F.Cu) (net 6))
 (segment (start 71.12 85.725) (end 67.945 88.9) (width 0.5) (layer B.Cu) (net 8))
 (segment (start 68.58 97.155) (end 69.85 97.155) (width 0.5) (layer B.Cu) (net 8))
 (segment (start 67.945 96.52) (end 68.58 97.155) (width 0.5) (layer B.Cu) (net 8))
 (segment (start 67.945 95.885) (end 67.945 96.52) (width 0.5) (layer B.Cu) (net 8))
 (segment (start 67.945 88.9) (end 67.945 95.885) (width 0.5) (layer B.Cu) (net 8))
 (segment (start 65.405 89.615) (end 66.12 89.615) (width 0.5) (layer F.Cu) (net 8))
 (segment (start 66.12 89.615) (end 67.945 91.44) (width 0.5) (layer F.Cu) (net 8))
 (segment (start 67.945 91.44) (end 67.945 96.52) (width 0.5) (layer F.Cu) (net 8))
 (segment (start 67.945 96.52) (end 68.58 97.155) (width 0.5) (layer F.Cu) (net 8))
 (segment (start 68.58 97.155) (end 69.85 97.155) (width 0.5) (layer F.Cu) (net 8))
 (segment (start 71.12 85.725) (end 70.485 85.725) (width 0.5) (layer B.Cu) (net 8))
 (segment (start 59.69 74.295) (end 58.42 74.295) (width 0.5) (layer F.Cu) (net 4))
 (segment (start 58.42 74.295) (end 57.785 74.93) (width 0.5) (layer F.Cu) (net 4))
 (segment (start 46.355 83.82) (end 46.355 85.645) (width 0.5) (layer F.Cu) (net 4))
 (segment (start 48.895 81.28) (end 46.355 83.82) (width 0.5) (layer F.Cu) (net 4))
 (segment (start 54.61 81.28) (end 48.895 81.28) (width 0.5) (layer F.Cu) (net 4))
 (segment (start 57.785 78.105) (end 54.61 81.28) (width 0.5) (layer F.Cu) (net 4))
 (segment (start 57.785 74.93) (end 57.785 78.105) (width 0.5) (layer F.Cu) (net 4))
 (segment (start 43.18 85.725) (end 46.275 85.725) (width 0.5) (layer F.Cu) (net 4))
 (segment (start 46.275 85.725) (end 46.355 85.645) (width 0.5) (layer F.Cu) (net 4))
 (segment (start 59.69 74.295) (end 59.055 74.295) (width 0.5) (layer F.Cu) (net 4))
 (segment (start 55.88 71.755) (end 54.61 71.755) (width 0.5) (layer F.Cu) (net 4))
 (segment (start 58.42 74.295) (end 55.88 71.755) (width 0.5) (layer F.Cu) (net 4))
 (segment (start 43.18 88.265) (end 46.275 88.265) (width 0.5) (layer F.Cu) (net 5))
 (segment (start 46.275 88.265) (end 46.355 88.345) (width 0.5) (layer F.Cu) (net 5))
 (segment (start 50.165 83.185) (end 55.245 83.185) (width 0.5) (layer B.Cu) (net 2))
 (segment (start 55.245 83.185) (end 66.04 93.98) (width 0.5) (layer B.Cu) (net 2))
 (segment (start 66.04 93.98) (end 66.04 100.48) (width 0.5) (layer F.Cu) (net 2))
 (via (at 50.165 83.185) (size 0.6858) (drill 0.3302) (layers F.Cu B.Cu) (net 2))
 (segment (start 50.165 83.185) (end 48.895 84.455) (width 0.5) (layer F.Cu) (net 2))
 (segment (start 48.895 84.455) (end 48.895 85.01) (width 0.5) (layer F.Cu) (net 2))
 (segment (start 47.625 80.645) (end 43.18 80.645) (width 0.5) (layer B.Cu) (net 2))
 (segment (start 50.165 83.185) (end 47.625 80.645) (width 0.5) (layer B.Cu) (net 2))
 (segment (start 43.815 93.83) (end 43.838 93.83) (width 0.5) (layer B.Cu) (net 1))
 (segment (start 43.838 93.83) (end 44.704 92.964) (width 0.5) (layer B.Cu) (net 1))
 (segment (start 44.704 92.964) (end 44.704 81.788) (width 0.5) (layer B.Cu) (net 1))
 (via (at 44.704 81.788) (size 0.6858) (drill 0.3302) (layers F.Cu B.Cu) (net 1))
 (segment (start 44.704 81.788) (end 44.704 76.2) (width 0.5) (layer F.Cu) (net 1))
 (segment (start 44.704 76.2) (end 44.704 74.676) (width 0.5) (layer F.Cu) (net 1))
 (segment (start 44.704 74.676) (end 43.18 73.152) (width 0.5) (layer F.Cu) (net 1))
 (segment (start 43.18 73.152) (end 43.18 73.025) (width 0.5) (layer F.Cu) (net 1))
 (segment (start 43.18 93.83) (end 43.18 100.33) (width 0.5) (layer B.Cu) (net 1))
 (segment (start 43.18 93.83) (end 43.33 93.83) (width 0.5) (layer B.Cu) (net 1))
 (segment (start 54.61 74.295) (end 55.88 74.295) (width 0.5) (layer F.Cu) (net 3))
 (segment (start 45.72 83.185) (end 43.18 83.185) (width 0.5) (layer F.Cu) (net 3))
 (segment (start 48.895 80.01) (end 45.72 83.185) (width 0.5) (layer F.Cu) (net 3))
 (segment (start 54.61 80.01) (end 48.895 80.01) (width 0.5) (layer F.Cu) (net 3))
 (segment (start 56.515 78.105) (end 54.61 80.01) (width 0.5) (layer F.Cu) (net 3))
 (segment (start 56.515 74.93) (end 56.515 78.105) (width 0.5) (layer F.Cu) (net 3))
 (segment (start 55.88 74.295) (end 56.515 74.93) (width 0.5) (layer F.Cu) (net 3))
 (segment (start 54.61 74.295) (end 55.245 74.295) (width 0.5) (layer F.Cu) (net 3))
 (segment (start 54.61 74.295) (end 55.88 74.295) (width 0.5) (layer B.Cu) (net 3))
 (segment (start 58.42 71.755) (end 59.69 71.755) (width 0.5) (layer B.Cu) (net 3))
 (segment (start 55.88 74.295) (end 58.42 71.755) (width 0.5) (layer B.Cu) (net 3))
 (segment (start 59.69 69.215) (end 62.23 69.215) (width 0.5) (layer B.Cu) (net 10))
 (segment (start 65.405 80.645) (end 71.12 80.645) (width 0.5) (layer B.Cu) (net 10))
 (segment (start 63.5 78.74) (end 65.405 80.645) (width 0.5) (layer B.Cu) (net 10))
 (segment (start 63.5 70.485) (end 63.5 78.74) (width 0.5) (layer B.Cu) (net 10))
 (segment (start 62.23 69.215) (end 63.5 70.485) (width 0.5) (layer B.Cu) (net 10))
 (segment (start 71.12 78.105) (end 69.85 78.105) (width 0.5) (layer B.Cu) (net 11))
 (segment (start 52.705 76.835) (end 54.61 76.835) (width 0.5) (layer B.Cu) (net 11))
 (segment (start 51.435 75.565) (end 52.705 76.835) (width 0.5) (layer B.Cu) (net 11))
 (segment (start 51.435 67.945) (end 51.435 75.565) (width 0.5) (layer B.Cu) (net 11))
 (segment (start 52.705 66.675) (end 51.435 67.945) (width 0.5) (layer B.Cu) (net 11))
 (segment (start 61.595 66.675) (end 52.705 66.675) (width 0.5) (layer B.Cu) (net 11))
 (segment (start 64.77 69.85) (end 61.595 66.675) (width 0.5) (layer B.Cu) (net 11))
 (segment (start 64.77 78.105) (end 64.77 69.85) (width 0.5) (layer B.Cu) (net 11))
 (segment (start 66.04 79.375) (end 64.77 78.105) (width 0.5) (layer B.Cu) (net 11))
 (segment (start 68.58 79.375) (end 66.04 79.375) (width 0.5) (layer B.Cu) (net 11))
 (segment (start 69.85 78.105) (end 68.58 79.375) (width 0.5) (layer B.Cu) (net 11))
 (segment (start 71.12 73.025) (end 71.12 64.008) (width 0.5) (layer B.Cu) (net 12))
 (segment (start 71.12 64.008) (end 69.342 62.23) (width 0.5) (layer B.Cu) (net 12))
 (segment (start 69.342 62.23) (end 68.58 62.23) (width 0.5) (layer B.Cu) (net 12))
 (segment (start 67.31 71.755) (end 67.691 71.755) (width 0.5) (layer F.Cu) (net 15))
 (segment (start 67.691 71.755) (end 69.596 69.85) (width 0.5) (layer F.Cu) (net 15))
 (segment (start 69.596 69.85) (end 69.596 68.58) (width 0.5) (layer F.Cu) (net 15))
 (segment (start 69.596 68.58) (end 67.31 66.294) (width 0.5) (layer F.Cu) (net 15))
 (segment (start 67.31 66.294) (end 54.356 66.294) (width 0.5) (layer F.Cu) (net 15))
 (segment (start 54.356 66.294) (end 48.895 71.755) (width 0.5) (layer F.Cu) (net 15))
 (segment (start 48.895 71.755) (end 46.99 71.755) (width 0.5) (layer F.Cu) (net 15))
 (segment (start 46.99 65.405) (end 46.355 66.04) (width 0.5) (layer F.Cu) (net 9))
 (segment (start 46.355 66.04) (end 43.895 66.04) (width 0.5) (layer F.Cu) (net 9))
 (segment (start 43.895 66.04) (end 43.815 65.96) (width 0.5) (layer F.Cu) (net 9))
 (segment (start 71.12 83.185) (end 59.055 83.185) (width 0.5) (layer B.Cu) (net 9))
 (segment (start 47.27 65.125) (end 47.27 62.775) (width 0.5) (layer F.Cu) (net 9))
 (segment (start 46.99 65.405) (end 47.27 65.125) (width 0.5) (layer F.Cu) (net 9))
 (via (at 46.99 65.405) (size 0.6858) (drill 0.3302) (layers F.Cu B.Cu) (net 9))
 (segment (start 45.085 67.31) (end 46.99 65.405) (width 0.5) (layer B.Cu) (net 9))
 (segment (start 45.085 78.105) (end 45.085 67.31) (width 0.5) (layer B.Cu) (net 9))
 (segment (start 46.355 79.375) (end 45.085 78.105) (width 0.5) (layer B.Cu) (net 9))
 (segment (start 55.245 79.375) (end 46.355 79.375) (width 0.5) (layer B.Cu) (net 9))
 (segment (start 59.055 83.185) (end 55.245 79.375) (width 0.5) (layer B.Cu) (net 9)))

